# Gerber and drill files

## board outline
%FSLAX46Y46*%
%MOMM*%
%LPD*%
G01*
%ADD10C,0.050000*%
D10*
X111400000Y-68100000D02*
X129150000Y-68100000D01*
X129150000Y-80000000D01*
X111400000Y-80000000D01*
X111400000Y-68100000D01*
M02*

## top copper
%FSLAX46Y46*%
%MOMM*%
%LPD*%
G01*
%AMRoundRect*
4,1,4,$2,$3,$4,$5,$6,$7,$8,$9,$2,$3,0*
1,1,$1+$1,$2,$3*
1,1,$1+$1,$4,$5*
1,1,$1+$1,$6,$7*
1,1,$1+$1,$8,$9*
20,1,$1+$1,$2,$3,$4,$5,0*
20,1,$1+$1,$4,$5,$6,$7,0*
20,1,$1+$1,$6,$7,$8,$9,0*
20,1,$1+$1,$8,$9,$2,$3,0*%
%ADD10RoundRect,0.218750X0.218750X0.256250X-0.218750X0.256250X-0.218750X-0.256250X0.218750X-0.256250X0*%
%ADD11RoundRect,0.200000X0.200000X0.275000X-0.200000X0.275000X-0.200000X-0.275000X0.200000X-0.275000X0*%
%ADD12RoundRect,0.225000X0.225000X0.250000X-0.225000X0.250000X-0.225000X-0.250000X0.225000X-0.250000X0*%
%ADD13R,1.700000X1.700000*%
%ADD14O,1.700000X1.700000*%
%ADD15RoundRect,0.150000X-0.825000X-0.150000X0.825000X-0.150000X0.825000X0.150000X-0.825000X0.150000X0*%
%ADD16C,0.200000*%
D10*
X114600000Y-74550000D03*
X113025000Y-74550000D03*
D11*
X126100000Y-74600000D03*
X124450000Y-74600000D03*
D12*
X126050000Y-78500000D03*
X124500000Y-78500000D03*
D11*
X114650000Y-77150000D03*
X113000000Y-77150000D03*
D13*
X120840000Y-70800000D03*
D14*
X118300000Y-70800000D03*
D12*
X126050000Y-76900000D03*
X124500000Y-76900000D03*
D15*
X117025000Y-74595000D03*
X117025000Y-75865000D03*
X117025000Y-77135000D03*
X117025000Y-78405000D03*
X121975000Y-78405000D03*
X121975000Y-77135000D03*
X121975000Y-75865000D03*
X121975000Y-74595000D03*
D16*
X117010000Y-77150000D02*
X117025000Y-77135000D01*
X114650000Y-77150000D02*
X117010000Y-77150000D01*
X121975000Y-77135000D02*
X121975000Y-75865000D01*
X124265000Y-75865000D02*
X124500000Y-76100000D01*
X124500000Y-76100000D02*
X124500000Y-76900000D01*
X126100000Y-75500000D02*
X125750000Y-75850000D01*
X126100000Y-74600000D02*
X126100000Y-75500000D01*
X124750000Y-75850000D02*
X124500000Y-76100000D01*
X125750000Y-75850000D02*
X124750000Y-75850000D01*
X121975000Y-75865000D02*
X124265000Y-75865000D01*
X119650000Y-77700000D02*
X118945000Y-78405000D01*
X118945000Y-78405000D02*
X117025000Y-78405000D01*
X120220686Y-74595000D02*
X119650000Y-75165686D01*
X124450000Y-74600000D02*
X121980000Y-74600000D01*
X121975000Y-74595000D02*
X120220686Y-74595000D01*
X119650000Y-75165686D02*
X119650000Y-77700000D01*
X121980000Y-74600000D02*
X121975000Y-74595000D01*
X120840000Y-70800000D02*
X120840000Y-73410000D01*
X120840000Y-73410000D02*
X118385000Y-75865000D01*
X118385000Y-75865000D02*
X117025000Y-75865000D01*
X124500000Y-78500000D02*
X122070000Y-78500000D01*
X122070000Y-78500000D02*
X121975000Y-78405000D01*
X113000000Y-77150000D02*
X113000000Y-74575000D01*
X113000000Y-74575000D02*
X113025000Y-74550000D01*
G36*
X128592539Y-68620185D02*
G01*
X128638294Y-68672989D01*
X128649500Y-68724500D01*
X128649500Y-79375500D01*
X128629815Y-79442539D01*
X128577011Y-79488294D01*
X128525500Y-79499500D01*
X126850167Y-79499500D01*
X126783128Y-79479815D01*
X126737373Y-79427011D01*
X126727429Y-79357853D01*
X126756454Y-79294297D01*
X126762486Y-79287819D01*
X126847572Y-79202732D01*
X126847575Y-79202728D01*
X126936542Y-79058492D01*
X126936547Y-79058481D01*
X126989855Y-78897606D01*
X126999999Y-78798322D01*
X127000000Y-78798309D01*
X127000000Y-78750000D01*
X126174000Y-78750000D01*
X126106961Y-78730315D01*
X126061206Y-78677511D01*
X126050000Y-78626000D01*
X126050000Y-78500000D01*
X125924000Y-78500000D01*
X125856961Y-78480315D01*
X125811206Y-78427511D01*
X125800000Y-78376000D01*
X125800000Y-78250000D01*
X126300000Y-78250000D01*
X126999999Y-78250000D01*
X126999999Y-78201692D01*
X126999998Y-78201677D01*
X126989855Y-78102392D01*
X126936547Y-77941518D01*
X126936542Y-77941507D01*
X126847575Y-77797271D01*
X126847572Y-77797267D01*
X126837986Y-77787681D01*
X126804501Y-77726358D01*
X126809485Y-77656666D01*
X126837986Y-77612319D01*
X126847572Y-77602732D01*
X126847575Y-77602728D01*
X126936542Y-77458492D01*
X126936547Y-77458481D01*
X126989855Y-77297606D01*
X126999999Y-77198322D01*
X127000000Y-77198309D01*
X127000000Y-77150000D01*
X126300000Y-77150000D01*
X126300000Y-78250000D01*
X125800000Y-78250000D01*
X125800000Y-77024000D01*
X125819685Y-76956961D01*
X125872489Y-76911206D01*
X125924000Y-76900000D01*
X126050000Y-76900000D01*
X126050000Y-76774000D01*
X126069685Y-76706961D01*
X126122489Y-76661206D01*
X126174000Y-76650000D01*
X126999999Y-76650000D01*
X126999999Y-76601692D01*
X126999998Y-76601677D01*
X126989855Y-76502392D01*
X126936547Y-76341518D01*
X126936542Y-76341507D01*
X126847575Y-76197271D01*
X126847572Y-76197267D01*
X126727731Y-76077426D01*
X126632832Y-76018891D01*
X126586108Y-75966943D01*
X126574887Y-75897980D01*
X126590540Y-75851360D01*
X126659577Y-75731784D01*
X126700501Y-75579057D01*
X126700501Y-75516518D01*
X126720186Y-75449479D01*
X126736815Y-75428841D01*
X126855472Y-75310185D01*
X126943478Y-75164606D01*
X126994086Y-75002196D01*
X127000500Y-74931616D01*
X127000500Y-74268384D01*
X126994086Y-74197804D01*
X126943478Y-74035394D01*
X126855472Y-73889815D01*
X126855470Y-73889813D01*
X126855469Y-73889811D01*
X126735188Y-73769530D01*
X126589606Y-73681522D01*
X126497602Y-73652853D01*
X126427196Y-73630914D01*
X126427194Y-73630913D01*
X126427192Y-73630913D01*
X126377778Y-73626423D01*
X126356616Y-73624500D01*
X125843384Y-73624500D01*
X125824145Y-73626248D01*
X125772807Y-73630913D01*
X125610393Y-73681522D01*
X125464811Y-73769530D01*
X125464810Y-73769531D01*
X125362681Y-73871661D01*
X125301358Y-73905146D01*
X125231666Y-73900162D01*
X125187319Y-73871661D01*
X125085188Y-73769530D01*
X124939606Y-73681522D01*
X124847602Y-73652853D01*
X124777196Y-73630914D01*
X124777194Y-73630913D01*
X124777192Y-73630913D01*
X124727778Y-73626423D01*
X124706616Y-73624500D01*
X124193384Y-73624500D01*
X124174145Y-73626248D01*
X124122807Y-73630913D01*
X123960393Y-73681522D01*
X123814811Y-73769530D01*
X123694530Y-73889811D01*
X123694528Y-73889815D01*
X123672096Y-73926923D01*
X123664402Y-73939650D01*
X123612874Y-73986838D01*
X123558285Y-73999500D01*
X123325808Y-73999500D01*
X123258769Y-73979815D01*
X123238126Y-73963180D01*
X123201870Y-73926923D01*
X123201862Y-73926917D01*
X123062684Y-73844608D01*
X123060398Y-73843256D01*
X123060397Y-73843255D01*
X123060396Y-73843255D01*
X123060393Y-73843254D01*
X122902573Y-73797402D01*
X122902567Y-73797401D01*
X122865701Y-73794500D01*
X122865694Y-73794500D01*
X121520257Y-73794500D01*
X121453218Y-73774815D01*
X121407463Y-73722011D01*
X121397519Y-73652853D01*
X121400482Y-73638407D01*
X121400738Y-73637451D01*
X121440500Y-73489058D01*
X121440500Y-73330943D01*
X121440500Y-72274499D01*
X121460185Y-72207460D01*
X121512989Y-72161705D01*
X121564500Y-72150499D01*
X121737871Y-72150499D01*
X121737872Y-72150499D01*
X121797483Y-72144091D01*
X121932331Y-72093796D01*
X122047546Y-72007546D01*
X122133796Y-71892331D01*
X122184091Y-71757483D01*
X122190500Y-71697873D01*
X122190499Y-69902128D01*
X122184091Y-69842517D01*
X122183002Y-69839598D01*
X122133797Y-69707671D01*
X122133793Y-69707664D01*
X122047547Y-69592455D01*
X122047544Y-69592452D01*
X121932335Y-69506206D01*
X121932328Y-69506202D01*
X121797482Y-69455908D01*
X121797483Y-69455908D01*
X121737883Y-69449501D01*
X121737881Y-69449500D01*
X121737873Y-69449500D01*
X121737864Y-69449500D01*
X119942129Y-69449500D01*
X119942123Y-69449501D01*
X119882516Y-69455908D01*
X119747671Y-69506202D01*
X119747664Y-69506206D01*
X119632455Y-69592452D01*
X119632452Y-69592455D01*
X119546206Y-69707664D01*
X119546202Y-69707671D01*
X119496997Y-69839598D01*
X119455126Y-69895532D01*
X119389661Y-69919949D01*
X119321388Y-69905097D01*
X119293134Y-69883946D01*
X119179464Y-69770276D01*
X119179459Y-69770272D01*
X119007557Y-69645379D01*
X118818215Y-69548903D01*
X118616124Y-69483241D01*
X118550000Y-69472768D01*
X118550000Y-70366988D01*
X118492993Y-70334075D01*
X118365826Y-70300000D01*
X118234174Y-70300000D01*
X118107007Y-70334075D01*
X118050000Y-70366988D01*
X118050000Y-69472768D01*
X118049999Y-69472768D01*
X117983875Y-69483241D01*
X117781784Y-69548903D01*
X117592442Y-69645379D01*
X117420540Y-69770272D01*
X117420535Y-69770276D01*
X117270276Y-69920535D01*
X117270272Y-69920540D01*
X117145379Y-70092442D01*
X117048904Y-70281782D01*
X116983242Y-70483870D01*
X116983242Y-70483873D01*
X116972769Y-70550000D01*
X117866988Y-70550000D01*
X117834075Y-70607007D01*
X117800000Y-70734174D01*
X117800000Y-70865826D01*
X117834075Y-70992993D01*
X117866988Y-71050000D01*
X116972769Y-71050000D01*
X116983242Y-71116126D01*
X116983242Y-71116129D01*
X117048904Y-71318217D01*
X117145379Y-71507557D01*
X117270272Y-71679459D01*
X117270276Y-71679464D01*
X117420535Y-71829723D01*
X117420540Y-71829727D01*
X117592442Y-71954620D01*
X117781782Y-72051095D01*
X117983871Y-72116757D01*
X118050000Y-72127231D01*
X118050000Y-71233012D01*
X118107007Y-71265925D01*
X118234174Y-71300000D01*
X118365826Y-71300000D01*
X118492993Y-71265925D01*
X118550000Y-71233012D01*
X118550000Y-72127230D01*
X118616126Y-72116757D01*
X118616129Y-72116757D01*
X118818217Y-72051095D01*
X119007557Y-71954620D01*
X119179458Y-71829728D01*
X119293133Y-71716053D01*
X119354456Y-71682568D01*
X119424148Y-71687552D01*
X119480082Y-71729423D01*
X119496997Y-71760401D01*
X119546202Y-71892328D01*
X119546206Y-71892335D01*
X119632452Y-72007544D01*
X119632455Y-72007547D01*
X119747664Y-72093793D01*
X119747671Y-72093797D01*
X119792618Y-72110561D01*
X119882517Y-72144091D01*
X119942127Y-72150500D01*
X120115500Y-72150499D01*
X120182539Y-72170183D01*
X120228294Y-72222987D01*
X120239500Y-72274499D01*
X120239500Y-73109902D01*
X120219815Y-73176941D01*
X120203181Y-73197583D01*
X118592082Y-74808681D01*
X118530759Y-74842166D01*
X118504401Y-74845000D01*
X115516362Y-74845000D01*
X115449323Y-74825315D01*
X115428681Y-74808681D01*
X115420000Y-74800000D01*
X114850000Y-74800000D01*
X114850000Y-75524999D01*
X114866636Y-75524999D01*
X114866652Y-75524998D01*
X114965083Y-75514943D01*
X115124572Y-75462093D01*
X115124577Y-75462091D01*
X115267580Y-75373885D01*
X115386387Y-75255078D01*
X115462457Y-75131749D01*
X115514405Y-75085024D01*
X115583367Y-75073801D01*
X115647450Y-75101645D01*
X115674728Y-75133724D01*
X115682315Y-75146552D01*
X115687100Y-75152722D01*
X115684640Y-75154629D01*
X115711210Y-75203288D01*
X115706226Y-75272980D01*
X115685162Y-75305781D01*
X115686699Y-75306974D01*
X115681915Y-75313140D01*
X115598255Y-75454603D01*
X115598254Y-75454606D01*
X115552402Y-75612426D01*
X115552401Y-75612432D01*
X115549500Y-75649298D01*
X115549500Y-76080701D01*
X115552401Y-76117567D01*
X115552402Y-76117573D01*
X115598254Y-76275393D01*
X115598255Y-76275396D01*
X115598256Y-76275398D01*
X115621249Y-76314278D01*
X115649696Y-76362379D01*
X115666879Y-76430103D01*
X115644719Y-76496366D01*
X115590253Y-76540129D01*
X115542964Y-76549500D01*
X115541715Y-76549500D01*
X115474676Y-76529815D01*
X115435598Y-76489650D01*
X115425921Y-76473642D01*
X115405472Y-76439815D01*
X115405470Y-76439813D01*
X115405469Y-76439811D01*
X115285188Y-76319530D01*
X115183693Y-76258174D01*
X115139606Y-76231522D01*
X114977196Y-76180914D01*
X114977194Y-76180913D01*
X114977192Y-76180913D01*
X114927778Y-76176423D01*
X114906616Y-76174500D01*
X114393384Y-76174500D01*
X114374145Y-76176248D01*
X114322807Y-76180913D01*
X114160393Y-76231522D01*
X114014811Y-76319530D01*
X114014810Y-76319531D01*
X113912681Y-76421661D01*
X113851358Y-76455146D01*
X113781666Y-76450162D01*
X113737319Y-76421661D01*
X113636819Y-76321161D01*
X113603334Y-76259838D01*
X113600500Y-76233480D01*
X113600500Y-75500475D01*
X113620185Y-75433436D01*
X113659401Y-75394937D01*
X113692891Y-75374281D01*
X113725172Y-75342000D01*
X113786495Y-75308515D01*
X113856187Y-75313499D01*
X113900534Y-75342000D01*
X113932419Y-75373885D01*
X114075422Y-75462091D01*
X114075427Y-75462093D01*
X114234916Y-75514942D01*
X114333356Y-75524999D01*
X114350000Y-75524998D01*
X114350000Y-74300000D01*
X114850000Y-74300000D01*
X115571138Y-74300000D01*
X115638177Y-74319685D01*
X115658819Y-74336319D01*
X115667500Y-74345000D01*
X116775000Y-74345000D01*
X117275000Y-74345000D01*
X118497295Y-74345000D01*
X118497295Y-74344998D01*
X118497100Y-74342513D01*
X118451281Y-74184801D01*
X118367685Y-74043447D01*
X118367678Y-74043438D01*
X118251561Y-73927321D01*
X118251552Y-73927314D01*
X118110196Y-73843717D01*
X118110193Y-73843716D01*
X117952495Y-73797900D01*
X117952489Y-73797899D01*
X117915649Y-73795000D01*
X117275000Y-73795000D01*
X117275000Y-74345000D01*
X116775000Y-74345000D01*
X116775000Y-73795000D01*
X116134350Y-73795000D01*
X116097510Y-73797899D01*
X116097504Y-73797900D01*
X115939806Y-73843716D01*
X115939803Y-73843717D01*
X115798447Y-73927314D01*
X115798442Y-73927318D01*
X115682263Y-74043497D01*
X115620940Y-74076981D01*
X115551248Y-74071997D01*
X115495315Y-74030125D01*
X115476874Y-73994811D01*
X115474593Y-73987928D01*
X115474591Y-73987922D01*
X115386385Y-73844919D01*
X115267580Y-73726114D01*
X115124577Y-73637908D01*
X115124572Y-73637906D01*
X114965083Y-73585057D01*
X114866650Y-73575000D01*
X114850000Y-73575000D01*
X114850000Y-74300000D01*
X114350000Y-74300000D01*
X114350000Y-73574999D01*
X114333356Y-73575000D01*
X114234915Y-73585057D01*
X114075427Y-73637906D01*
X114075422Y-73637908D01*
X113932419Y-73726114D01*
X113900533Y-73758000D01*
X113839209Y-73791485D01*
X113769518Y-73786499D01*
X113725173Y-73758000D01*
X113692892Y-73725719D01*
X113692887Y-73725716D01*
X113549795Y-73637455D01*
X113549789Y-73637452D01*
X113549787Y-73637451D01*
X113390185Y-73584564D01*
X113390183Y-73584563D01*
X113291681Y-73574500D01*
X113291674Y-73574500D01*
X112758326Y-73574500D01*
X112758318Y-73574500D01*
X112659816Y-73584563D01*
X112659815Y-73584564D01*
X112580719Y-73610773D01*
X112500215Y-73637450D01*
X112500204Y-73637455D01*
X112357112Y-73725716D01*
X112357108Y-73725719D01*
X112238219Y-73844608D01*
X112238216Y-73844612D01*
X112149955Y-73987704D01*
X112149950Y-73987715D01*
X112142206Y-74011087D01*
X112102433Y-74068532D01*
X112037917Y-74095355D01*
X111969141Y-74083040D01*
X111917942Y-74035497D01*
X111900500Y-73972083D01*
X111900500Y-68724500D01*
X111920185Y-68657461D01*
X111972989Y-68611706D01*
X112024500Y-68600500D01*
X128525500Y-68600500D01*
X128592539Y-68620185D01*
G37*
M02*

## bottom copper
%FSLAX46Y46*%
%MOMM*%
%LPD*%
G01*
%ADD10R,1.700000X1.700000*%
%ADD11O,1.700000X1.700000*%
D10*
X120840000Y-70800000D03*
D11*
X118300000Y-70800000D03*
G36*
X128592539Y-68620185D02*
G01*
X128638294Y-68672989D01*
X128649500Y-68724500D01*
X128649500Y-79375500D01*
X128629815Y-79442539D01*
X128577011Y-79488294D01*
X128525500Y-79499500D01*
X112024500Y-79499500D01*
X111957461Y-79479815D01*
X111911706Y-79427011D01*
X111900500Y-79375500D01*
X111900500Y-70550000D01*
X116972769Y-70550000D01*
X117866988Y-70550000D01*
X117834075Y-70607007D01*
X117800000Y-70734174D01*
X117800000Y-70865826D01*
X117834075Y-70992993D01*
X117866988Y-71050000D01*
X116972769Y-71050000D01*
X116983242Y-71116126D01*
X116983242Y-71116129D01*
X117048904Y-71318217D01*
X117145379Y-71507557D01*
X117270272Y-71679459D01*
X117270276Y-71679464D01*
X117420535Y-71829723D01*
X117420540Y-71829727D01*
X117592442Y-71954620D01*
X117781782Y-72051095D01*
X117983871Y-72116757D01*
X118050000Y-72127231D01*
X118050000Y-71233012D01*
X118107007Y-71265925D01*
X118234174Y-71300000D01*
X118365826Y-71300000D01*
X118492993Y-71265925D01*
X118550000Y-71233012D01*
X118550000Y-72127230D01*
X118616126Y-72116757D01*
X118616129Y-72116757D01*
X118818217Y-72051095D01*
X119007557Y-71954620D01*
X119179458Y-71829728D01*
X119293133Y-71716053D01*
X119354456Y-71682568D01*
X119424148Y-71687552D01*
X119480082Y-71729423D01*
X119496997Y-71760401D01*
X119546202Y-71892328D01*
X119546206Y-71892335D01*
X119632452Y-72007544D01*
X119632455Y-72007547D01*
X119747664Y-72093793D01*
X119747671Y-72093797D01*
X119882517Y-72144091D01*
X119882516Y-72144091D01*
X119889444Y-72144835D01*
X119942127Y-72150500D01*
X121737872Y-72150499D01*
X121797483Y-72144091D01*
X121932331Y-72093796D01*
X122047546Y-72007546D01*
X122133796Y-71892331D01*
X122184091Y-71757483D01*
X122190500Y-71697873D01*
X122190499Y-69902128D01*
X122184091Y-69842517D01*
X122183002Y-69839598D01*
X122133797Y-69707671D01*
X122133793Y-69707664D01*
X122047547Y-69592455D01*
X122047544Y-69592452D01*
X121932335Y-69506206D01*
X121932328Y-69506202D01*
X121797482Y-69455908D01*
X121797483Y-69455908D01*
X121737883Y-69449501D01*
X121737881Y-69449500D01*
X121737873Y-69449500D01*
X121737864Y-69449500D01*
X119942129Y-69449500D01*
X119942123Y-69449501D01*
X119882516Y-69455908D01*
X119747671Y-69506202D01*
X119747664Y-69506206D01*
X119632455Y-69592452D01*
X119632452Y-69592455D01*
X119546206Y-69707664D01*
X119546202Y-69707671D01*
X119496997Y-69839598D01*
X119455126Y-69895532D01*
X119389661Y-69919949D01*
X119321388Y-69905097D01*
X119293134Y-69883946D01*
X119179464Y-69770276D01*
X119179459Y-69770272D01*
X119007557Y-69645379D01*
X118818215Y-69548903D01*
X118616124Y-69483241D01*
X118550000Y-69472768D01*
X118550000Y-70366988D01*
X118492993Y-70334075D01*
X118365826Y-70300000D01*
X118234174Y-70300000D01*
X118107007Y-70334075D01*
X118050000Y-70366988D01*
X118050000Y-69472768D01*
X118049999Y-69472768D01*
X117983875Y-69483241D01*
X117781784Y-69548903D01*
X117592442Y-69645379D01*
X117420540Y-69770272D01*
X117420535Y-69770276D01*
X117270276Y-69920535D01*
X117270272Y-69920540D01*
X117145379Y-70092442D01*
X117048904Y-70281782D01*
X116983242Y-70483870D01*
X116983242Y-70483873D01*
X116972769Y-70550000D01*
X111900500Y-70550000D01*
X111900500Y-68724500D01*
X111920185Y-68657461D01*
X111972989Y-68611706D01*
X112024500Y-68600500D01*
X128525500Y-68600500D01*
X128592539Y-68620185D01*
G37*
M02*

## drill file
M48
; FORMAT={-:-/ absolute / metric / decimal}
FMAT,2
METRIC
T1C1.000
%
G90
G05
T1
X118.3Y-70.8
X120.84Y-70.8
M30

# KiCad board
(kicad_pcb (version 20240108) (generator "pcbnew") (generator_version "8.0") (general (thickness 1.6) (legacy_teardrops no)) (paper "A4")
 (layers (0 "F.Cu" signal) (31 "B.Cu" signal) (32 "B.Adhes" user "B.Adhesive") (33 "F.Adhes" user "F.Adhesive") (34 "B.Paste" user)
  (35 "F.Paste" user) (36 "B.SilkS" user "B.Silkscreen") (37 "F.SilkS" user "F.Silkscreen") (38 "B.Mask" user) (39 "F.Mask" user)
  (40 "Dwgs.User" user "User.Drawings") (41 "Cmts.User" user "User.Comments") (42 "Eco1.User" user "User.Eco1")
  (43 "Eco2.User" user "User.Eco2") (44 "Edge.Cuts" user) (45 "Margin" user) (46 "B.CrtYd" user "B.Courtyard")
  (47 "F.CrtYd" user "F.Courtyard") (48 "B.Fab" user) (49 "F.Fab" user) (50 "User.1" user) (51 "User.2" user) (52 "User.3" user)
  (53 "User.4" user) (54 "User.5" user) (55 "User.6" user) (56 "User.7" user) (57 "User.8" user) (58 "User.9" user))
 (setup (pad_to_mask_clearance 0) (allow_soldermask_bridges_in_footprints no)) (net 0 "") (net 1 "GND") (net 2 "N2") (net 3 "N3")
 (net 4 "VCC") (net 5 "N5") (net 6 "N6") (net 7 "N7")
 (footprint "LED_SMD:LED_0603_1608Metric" (layer "F.Cu") (at 113.8125 74.55 180)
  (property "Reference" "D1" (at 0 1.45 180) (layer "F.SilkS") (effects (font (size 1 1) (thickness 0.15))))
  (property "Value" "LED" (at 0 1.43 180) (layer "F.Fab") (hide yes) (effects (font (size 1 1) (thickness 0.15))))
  (pad "1" smd roundrect (at -0.7875 0 180) (size 0.875 0.95) (layers "F.Cu" "F.Paste" "F.Mask") (roundrect_rratio 0.25) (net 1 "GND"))
  (pad "2" smd roundrect (at 0.7875 0 180) (size 0.875 0.95) (layers "F.Cu" "F.Paste" "F.Mask") (roundrect_rratio 0.25) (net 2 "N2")))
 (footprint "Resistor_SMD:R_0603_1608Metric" (layer "F.Cu") (at 125.275 74.6 180)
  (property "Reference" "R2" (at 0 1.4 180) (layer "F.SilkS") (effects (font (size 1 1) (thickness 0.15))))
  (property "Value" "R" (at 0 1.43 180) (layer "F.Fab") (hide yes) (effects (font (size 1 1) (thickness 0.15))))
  (pad "1" smd roundrect (at -0.825 0 180) (size 0.8 0.95) (layers "F.Cu" "F.Paste" "F.Mask") (roundrect_rratio 0.25) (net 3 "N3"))
  (pad "2" smd roundrect (at 0.825 0 180) (size 0.8 0.95) (layers "F.Cu" "F.Paste" "F.Mask") (roundrect_rratio 0.25) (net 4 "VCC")))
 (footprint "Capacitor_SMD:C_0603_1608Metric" (layer "F.Cu") (at 125.275 78.5 180)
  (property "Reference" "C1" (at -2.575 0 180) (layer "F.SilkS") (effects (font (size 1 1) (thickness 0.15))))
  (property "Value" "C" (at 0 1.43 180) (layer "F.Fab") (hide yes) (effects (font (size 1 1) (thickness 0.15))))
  (pad "1" smd roundrect (at -0.775 0 180) (size 0.9 0.95) (layers "F.Cu" "F.Paste" "F.Mask") (roundrect_rratio 0.25) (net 1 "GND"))
  (pad "2" smd roundrect (at 0.775 0 180) (size 0.9 0.95) (layers "F.Cu" "F.Paste" "F.Mask") (roundrect_rratio 0.25) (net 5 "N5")))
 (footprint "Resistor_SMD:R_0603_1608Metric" (layer "F.Cu") (at 113.825 77.15 180)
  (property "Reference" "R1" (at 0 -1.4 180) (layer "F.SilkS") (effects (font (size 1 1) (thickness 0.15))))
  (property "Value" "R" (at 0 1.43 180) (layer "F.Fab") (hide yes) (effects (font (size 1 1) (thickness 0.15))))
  (pad "1" smd roundrect (at -0.825 0 180) (size 0.8 0.95) (layers "F.Cu" "F.Paste" "F.Mask") (roundrect_rratio 0.25) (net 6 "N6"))
  (pad "2" smd roundrect (at 0.825 0 180) (size 0.8 0.95) (layers "F.Cu" "F.Paste" "F.Mask") (roundrect_rratio 0.25) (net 2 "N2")))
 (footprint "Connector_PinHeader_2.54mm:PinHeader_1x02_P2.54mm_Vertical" (layer "F.Cu") (at 120.84 70.8 -90)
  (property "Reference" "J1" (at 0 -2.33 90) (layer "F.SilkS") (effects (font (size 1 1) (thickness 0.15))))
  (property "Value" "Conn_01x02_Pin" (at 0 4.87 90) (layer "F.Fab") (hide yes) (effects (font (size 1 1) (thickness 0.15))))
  (pad "1" thru_hole rect (at 0 0 270) (size 1.7 1.7) (drill 1) (layers "*.Cu" "*.Mask") (remove_unused_layers no) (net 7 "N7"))
  (pad "2" thru_hole oval (at 0 2.54 270) (size 1.7 1.7) (drill 1) (layers "*.Cu" "*.Mask") (remove_unused_layers no) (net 1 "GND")))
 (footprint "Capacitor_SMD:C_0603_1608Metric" (layer "F.Cu") (at 125.275 76.9 180)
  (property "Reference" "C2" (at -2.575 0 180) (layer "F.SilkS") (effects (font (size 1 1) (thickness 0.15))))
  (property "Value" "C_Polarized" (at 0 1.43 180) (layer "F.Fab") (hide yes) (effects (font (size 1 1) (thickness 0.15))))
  (pad "1" smd roundrect (at -0.775 0 180) (size 0.9 0.95) (layers "F.Cu" "F.Paste" "F.Mask") (roundrect_rratio 0.25) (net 1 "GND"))
  (pad "2" smd roundrect (at 0.775 0 180) (size 0.9 0.95) (layers "F.Cu" "F.Paste" "F.Mask") (roundrect_rratio 0.25) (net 3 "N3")))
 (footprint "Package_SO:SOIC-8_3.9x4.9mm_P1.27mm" (layer "F.Cu") (at 119.5 76.5)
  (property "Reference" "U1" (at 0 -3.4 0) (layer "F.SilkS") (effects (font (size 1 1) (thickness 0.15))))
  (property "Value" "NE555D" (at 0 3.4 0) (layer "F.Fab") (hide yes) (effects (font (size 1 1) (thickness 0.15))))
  (pad "1" smd roundrect (at -2.475 -1.905) (size 1.95 0.6) (layers "F.Cu" "F.Paste" "F.Mask") (roundrect_rratio 0.25) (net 1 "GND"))
  (pad "2" smd roundrect (at -2.475 -0.635) (size 1.95 0.6) (layers "F.Cu" "F.Paste" "F.Mask") (roundrect_rratio 0.25) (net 7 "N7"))
  (pad "3" smd roundrect (at -2.475 0.635) (size 1.95 0.6) (layers "F.Cu" "F.Paste" "F.Mask") (roundrect_rratio 0.25) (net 6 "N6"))
  (pad "4" smd roundrect (at -2.475 1.905) (size 1.95 0.6) (layers "F.Cu" "F.Paste" "F.Mask") (roundrect_rratio 0.25) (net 4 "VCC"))
  (pad "5" smd roundrect (at 2.475 1.905) (size 1.95 0.6) (layers "F.Cu" "F.Paste" "F.Mask") (roundrect_rratio 0.25) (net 5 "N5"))
  (pad "6" smd roundrect (at 2.475 0.635) (size 1.95 0.6) (layers "F.Cu" "F.Paste" "F.Mask") (roundrect_rratio 0.25) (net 3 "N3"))
  (pad "7" smd roundrect (at 2.475 -0.635) (size 1.95 0.6) (layers "F.Cu" "F.Paste" "F.Mask") (roundrect_rratio 0.25) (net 3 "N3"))
  (pad "8" smd roundrect (at 2.475 -1.905) (size 1.95 0.6) (layers "F.Cu" "F.Paste" "F.Mask") (roundrect_rratio 0.25) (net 4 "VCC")))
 (gr_rect (start 111.4 68.1) (end 129.15 80) (stroke (width 0.05) (type default)) (fill none) (layer "Edge.Cuts"))
 (segment (start 117.01 77.15) (end 117.025 77.135) (width 0.2) (layer "F.Cu") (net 6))
 (segment (start 114.65 77.15) (end 117.01 77.15) (width 0.2) (layer "F.Cu") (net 6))
 (segment (start 121.975 77.135) (end 121.975 75.865) (width 0.2) (layer "F.Cu") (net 3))
 (segment (start 124.265 75.865) (end 124.5 76.1) (width 0.2) (layer "F.Cu") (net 3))
 (segment (start 124.5 76.1) (end 124.5 76.9) (width 0.2) (layer "F.Cu") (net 3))
 (segment (start 126.1 75.5) (end 125.75 75.85) (width 0.2) (layer "F.Cu") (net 3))
 (segment (start 126.1 74.6) (end 126.1 75.5) (width 0.2) (layer "F.Cu") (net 3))
 (segment (start 124.75 75.85) (end 124.5 76.1) (width 0.2) (layer "F.Cu") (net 3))
 (segment (start 125.75 75.85) (end 124.75 75.85) (width 0.2) (layer "F.Cu") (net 3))
 (segment (start 121.975 75.865) (end 124.265 75.865) (width 0.2) (layer "F.Cu") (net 3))
 (segment (start 119.65 77.7) (end 118.945 78.405) (width 0.2) (layer "F.Cu") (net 4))
 (segment (start 118.945 78.405) (end 117.025 78.405) (width 0.2) (layer "F.Cu") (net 4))
 (segment (start 120.220686 74.595) (end 119.65 75.165686) (width 0.2) (layer "F.Cu") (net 4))
 (segment (start 124.45 74.6) (end 121.98 74.6) (width 0.2) (layer "F.Cu") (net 4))
 (segment (start 121.975 74.595) (end 120.220686 74.595) (width 0.2) (layer "F.Cu") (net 4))
 (segment (start 119.65 75.165686) (end 119.65 77.7) (width 0.2) (layer "F.Cu") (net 4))
 (segment (start 121.98 74.6) (end 121.975 74.595) (width 0.2) (layer "F.Cu") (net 4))
 (segment (start 120.84 70.8) (end 120.84 73.41) (width 0.2) (layer "F.Cu") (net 7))
 (segment (start 120.84 73.41) (end 118.385 75.865) (width 0.2) (layer "F.Cu") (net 7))
 (segment (start 118.385 75.865) (end 117.025 75.865) (width 0.2) (layer "F.Cu") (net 7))
 (segment (start 124.5 78.5) (end 122.07 78.5) (width 0.2) (layer "F.Cu") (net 5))
 (segment (start 122.07 78.5) (end 121.975 78.405) (width 0.2) (layer "F.Cu") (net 5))
 (segment (start 113 77.15) (end 113 74.575) (width 0.2) (layer "F.Cu") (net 2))
 (segment (start 113 74.575) (end 113.025 74.55) (width 0.2) (layer "F.Cu") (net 2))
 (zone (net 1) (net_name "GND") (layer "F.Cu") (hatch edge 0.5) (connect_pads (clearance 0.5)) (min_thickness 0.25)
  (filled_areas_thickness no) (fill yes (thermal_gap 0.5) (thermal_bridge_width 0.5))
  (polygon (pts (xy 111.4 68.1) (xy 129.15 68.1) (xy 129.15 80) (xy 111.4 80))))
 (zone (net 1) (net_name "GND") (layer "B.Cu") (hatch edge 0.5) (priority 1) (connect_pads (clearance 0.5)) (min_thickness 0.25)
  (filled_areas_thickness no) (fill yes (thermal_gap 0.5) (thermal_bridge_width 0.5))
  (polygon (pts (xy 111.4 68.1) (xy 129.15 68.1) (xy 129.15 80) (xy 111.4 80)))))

